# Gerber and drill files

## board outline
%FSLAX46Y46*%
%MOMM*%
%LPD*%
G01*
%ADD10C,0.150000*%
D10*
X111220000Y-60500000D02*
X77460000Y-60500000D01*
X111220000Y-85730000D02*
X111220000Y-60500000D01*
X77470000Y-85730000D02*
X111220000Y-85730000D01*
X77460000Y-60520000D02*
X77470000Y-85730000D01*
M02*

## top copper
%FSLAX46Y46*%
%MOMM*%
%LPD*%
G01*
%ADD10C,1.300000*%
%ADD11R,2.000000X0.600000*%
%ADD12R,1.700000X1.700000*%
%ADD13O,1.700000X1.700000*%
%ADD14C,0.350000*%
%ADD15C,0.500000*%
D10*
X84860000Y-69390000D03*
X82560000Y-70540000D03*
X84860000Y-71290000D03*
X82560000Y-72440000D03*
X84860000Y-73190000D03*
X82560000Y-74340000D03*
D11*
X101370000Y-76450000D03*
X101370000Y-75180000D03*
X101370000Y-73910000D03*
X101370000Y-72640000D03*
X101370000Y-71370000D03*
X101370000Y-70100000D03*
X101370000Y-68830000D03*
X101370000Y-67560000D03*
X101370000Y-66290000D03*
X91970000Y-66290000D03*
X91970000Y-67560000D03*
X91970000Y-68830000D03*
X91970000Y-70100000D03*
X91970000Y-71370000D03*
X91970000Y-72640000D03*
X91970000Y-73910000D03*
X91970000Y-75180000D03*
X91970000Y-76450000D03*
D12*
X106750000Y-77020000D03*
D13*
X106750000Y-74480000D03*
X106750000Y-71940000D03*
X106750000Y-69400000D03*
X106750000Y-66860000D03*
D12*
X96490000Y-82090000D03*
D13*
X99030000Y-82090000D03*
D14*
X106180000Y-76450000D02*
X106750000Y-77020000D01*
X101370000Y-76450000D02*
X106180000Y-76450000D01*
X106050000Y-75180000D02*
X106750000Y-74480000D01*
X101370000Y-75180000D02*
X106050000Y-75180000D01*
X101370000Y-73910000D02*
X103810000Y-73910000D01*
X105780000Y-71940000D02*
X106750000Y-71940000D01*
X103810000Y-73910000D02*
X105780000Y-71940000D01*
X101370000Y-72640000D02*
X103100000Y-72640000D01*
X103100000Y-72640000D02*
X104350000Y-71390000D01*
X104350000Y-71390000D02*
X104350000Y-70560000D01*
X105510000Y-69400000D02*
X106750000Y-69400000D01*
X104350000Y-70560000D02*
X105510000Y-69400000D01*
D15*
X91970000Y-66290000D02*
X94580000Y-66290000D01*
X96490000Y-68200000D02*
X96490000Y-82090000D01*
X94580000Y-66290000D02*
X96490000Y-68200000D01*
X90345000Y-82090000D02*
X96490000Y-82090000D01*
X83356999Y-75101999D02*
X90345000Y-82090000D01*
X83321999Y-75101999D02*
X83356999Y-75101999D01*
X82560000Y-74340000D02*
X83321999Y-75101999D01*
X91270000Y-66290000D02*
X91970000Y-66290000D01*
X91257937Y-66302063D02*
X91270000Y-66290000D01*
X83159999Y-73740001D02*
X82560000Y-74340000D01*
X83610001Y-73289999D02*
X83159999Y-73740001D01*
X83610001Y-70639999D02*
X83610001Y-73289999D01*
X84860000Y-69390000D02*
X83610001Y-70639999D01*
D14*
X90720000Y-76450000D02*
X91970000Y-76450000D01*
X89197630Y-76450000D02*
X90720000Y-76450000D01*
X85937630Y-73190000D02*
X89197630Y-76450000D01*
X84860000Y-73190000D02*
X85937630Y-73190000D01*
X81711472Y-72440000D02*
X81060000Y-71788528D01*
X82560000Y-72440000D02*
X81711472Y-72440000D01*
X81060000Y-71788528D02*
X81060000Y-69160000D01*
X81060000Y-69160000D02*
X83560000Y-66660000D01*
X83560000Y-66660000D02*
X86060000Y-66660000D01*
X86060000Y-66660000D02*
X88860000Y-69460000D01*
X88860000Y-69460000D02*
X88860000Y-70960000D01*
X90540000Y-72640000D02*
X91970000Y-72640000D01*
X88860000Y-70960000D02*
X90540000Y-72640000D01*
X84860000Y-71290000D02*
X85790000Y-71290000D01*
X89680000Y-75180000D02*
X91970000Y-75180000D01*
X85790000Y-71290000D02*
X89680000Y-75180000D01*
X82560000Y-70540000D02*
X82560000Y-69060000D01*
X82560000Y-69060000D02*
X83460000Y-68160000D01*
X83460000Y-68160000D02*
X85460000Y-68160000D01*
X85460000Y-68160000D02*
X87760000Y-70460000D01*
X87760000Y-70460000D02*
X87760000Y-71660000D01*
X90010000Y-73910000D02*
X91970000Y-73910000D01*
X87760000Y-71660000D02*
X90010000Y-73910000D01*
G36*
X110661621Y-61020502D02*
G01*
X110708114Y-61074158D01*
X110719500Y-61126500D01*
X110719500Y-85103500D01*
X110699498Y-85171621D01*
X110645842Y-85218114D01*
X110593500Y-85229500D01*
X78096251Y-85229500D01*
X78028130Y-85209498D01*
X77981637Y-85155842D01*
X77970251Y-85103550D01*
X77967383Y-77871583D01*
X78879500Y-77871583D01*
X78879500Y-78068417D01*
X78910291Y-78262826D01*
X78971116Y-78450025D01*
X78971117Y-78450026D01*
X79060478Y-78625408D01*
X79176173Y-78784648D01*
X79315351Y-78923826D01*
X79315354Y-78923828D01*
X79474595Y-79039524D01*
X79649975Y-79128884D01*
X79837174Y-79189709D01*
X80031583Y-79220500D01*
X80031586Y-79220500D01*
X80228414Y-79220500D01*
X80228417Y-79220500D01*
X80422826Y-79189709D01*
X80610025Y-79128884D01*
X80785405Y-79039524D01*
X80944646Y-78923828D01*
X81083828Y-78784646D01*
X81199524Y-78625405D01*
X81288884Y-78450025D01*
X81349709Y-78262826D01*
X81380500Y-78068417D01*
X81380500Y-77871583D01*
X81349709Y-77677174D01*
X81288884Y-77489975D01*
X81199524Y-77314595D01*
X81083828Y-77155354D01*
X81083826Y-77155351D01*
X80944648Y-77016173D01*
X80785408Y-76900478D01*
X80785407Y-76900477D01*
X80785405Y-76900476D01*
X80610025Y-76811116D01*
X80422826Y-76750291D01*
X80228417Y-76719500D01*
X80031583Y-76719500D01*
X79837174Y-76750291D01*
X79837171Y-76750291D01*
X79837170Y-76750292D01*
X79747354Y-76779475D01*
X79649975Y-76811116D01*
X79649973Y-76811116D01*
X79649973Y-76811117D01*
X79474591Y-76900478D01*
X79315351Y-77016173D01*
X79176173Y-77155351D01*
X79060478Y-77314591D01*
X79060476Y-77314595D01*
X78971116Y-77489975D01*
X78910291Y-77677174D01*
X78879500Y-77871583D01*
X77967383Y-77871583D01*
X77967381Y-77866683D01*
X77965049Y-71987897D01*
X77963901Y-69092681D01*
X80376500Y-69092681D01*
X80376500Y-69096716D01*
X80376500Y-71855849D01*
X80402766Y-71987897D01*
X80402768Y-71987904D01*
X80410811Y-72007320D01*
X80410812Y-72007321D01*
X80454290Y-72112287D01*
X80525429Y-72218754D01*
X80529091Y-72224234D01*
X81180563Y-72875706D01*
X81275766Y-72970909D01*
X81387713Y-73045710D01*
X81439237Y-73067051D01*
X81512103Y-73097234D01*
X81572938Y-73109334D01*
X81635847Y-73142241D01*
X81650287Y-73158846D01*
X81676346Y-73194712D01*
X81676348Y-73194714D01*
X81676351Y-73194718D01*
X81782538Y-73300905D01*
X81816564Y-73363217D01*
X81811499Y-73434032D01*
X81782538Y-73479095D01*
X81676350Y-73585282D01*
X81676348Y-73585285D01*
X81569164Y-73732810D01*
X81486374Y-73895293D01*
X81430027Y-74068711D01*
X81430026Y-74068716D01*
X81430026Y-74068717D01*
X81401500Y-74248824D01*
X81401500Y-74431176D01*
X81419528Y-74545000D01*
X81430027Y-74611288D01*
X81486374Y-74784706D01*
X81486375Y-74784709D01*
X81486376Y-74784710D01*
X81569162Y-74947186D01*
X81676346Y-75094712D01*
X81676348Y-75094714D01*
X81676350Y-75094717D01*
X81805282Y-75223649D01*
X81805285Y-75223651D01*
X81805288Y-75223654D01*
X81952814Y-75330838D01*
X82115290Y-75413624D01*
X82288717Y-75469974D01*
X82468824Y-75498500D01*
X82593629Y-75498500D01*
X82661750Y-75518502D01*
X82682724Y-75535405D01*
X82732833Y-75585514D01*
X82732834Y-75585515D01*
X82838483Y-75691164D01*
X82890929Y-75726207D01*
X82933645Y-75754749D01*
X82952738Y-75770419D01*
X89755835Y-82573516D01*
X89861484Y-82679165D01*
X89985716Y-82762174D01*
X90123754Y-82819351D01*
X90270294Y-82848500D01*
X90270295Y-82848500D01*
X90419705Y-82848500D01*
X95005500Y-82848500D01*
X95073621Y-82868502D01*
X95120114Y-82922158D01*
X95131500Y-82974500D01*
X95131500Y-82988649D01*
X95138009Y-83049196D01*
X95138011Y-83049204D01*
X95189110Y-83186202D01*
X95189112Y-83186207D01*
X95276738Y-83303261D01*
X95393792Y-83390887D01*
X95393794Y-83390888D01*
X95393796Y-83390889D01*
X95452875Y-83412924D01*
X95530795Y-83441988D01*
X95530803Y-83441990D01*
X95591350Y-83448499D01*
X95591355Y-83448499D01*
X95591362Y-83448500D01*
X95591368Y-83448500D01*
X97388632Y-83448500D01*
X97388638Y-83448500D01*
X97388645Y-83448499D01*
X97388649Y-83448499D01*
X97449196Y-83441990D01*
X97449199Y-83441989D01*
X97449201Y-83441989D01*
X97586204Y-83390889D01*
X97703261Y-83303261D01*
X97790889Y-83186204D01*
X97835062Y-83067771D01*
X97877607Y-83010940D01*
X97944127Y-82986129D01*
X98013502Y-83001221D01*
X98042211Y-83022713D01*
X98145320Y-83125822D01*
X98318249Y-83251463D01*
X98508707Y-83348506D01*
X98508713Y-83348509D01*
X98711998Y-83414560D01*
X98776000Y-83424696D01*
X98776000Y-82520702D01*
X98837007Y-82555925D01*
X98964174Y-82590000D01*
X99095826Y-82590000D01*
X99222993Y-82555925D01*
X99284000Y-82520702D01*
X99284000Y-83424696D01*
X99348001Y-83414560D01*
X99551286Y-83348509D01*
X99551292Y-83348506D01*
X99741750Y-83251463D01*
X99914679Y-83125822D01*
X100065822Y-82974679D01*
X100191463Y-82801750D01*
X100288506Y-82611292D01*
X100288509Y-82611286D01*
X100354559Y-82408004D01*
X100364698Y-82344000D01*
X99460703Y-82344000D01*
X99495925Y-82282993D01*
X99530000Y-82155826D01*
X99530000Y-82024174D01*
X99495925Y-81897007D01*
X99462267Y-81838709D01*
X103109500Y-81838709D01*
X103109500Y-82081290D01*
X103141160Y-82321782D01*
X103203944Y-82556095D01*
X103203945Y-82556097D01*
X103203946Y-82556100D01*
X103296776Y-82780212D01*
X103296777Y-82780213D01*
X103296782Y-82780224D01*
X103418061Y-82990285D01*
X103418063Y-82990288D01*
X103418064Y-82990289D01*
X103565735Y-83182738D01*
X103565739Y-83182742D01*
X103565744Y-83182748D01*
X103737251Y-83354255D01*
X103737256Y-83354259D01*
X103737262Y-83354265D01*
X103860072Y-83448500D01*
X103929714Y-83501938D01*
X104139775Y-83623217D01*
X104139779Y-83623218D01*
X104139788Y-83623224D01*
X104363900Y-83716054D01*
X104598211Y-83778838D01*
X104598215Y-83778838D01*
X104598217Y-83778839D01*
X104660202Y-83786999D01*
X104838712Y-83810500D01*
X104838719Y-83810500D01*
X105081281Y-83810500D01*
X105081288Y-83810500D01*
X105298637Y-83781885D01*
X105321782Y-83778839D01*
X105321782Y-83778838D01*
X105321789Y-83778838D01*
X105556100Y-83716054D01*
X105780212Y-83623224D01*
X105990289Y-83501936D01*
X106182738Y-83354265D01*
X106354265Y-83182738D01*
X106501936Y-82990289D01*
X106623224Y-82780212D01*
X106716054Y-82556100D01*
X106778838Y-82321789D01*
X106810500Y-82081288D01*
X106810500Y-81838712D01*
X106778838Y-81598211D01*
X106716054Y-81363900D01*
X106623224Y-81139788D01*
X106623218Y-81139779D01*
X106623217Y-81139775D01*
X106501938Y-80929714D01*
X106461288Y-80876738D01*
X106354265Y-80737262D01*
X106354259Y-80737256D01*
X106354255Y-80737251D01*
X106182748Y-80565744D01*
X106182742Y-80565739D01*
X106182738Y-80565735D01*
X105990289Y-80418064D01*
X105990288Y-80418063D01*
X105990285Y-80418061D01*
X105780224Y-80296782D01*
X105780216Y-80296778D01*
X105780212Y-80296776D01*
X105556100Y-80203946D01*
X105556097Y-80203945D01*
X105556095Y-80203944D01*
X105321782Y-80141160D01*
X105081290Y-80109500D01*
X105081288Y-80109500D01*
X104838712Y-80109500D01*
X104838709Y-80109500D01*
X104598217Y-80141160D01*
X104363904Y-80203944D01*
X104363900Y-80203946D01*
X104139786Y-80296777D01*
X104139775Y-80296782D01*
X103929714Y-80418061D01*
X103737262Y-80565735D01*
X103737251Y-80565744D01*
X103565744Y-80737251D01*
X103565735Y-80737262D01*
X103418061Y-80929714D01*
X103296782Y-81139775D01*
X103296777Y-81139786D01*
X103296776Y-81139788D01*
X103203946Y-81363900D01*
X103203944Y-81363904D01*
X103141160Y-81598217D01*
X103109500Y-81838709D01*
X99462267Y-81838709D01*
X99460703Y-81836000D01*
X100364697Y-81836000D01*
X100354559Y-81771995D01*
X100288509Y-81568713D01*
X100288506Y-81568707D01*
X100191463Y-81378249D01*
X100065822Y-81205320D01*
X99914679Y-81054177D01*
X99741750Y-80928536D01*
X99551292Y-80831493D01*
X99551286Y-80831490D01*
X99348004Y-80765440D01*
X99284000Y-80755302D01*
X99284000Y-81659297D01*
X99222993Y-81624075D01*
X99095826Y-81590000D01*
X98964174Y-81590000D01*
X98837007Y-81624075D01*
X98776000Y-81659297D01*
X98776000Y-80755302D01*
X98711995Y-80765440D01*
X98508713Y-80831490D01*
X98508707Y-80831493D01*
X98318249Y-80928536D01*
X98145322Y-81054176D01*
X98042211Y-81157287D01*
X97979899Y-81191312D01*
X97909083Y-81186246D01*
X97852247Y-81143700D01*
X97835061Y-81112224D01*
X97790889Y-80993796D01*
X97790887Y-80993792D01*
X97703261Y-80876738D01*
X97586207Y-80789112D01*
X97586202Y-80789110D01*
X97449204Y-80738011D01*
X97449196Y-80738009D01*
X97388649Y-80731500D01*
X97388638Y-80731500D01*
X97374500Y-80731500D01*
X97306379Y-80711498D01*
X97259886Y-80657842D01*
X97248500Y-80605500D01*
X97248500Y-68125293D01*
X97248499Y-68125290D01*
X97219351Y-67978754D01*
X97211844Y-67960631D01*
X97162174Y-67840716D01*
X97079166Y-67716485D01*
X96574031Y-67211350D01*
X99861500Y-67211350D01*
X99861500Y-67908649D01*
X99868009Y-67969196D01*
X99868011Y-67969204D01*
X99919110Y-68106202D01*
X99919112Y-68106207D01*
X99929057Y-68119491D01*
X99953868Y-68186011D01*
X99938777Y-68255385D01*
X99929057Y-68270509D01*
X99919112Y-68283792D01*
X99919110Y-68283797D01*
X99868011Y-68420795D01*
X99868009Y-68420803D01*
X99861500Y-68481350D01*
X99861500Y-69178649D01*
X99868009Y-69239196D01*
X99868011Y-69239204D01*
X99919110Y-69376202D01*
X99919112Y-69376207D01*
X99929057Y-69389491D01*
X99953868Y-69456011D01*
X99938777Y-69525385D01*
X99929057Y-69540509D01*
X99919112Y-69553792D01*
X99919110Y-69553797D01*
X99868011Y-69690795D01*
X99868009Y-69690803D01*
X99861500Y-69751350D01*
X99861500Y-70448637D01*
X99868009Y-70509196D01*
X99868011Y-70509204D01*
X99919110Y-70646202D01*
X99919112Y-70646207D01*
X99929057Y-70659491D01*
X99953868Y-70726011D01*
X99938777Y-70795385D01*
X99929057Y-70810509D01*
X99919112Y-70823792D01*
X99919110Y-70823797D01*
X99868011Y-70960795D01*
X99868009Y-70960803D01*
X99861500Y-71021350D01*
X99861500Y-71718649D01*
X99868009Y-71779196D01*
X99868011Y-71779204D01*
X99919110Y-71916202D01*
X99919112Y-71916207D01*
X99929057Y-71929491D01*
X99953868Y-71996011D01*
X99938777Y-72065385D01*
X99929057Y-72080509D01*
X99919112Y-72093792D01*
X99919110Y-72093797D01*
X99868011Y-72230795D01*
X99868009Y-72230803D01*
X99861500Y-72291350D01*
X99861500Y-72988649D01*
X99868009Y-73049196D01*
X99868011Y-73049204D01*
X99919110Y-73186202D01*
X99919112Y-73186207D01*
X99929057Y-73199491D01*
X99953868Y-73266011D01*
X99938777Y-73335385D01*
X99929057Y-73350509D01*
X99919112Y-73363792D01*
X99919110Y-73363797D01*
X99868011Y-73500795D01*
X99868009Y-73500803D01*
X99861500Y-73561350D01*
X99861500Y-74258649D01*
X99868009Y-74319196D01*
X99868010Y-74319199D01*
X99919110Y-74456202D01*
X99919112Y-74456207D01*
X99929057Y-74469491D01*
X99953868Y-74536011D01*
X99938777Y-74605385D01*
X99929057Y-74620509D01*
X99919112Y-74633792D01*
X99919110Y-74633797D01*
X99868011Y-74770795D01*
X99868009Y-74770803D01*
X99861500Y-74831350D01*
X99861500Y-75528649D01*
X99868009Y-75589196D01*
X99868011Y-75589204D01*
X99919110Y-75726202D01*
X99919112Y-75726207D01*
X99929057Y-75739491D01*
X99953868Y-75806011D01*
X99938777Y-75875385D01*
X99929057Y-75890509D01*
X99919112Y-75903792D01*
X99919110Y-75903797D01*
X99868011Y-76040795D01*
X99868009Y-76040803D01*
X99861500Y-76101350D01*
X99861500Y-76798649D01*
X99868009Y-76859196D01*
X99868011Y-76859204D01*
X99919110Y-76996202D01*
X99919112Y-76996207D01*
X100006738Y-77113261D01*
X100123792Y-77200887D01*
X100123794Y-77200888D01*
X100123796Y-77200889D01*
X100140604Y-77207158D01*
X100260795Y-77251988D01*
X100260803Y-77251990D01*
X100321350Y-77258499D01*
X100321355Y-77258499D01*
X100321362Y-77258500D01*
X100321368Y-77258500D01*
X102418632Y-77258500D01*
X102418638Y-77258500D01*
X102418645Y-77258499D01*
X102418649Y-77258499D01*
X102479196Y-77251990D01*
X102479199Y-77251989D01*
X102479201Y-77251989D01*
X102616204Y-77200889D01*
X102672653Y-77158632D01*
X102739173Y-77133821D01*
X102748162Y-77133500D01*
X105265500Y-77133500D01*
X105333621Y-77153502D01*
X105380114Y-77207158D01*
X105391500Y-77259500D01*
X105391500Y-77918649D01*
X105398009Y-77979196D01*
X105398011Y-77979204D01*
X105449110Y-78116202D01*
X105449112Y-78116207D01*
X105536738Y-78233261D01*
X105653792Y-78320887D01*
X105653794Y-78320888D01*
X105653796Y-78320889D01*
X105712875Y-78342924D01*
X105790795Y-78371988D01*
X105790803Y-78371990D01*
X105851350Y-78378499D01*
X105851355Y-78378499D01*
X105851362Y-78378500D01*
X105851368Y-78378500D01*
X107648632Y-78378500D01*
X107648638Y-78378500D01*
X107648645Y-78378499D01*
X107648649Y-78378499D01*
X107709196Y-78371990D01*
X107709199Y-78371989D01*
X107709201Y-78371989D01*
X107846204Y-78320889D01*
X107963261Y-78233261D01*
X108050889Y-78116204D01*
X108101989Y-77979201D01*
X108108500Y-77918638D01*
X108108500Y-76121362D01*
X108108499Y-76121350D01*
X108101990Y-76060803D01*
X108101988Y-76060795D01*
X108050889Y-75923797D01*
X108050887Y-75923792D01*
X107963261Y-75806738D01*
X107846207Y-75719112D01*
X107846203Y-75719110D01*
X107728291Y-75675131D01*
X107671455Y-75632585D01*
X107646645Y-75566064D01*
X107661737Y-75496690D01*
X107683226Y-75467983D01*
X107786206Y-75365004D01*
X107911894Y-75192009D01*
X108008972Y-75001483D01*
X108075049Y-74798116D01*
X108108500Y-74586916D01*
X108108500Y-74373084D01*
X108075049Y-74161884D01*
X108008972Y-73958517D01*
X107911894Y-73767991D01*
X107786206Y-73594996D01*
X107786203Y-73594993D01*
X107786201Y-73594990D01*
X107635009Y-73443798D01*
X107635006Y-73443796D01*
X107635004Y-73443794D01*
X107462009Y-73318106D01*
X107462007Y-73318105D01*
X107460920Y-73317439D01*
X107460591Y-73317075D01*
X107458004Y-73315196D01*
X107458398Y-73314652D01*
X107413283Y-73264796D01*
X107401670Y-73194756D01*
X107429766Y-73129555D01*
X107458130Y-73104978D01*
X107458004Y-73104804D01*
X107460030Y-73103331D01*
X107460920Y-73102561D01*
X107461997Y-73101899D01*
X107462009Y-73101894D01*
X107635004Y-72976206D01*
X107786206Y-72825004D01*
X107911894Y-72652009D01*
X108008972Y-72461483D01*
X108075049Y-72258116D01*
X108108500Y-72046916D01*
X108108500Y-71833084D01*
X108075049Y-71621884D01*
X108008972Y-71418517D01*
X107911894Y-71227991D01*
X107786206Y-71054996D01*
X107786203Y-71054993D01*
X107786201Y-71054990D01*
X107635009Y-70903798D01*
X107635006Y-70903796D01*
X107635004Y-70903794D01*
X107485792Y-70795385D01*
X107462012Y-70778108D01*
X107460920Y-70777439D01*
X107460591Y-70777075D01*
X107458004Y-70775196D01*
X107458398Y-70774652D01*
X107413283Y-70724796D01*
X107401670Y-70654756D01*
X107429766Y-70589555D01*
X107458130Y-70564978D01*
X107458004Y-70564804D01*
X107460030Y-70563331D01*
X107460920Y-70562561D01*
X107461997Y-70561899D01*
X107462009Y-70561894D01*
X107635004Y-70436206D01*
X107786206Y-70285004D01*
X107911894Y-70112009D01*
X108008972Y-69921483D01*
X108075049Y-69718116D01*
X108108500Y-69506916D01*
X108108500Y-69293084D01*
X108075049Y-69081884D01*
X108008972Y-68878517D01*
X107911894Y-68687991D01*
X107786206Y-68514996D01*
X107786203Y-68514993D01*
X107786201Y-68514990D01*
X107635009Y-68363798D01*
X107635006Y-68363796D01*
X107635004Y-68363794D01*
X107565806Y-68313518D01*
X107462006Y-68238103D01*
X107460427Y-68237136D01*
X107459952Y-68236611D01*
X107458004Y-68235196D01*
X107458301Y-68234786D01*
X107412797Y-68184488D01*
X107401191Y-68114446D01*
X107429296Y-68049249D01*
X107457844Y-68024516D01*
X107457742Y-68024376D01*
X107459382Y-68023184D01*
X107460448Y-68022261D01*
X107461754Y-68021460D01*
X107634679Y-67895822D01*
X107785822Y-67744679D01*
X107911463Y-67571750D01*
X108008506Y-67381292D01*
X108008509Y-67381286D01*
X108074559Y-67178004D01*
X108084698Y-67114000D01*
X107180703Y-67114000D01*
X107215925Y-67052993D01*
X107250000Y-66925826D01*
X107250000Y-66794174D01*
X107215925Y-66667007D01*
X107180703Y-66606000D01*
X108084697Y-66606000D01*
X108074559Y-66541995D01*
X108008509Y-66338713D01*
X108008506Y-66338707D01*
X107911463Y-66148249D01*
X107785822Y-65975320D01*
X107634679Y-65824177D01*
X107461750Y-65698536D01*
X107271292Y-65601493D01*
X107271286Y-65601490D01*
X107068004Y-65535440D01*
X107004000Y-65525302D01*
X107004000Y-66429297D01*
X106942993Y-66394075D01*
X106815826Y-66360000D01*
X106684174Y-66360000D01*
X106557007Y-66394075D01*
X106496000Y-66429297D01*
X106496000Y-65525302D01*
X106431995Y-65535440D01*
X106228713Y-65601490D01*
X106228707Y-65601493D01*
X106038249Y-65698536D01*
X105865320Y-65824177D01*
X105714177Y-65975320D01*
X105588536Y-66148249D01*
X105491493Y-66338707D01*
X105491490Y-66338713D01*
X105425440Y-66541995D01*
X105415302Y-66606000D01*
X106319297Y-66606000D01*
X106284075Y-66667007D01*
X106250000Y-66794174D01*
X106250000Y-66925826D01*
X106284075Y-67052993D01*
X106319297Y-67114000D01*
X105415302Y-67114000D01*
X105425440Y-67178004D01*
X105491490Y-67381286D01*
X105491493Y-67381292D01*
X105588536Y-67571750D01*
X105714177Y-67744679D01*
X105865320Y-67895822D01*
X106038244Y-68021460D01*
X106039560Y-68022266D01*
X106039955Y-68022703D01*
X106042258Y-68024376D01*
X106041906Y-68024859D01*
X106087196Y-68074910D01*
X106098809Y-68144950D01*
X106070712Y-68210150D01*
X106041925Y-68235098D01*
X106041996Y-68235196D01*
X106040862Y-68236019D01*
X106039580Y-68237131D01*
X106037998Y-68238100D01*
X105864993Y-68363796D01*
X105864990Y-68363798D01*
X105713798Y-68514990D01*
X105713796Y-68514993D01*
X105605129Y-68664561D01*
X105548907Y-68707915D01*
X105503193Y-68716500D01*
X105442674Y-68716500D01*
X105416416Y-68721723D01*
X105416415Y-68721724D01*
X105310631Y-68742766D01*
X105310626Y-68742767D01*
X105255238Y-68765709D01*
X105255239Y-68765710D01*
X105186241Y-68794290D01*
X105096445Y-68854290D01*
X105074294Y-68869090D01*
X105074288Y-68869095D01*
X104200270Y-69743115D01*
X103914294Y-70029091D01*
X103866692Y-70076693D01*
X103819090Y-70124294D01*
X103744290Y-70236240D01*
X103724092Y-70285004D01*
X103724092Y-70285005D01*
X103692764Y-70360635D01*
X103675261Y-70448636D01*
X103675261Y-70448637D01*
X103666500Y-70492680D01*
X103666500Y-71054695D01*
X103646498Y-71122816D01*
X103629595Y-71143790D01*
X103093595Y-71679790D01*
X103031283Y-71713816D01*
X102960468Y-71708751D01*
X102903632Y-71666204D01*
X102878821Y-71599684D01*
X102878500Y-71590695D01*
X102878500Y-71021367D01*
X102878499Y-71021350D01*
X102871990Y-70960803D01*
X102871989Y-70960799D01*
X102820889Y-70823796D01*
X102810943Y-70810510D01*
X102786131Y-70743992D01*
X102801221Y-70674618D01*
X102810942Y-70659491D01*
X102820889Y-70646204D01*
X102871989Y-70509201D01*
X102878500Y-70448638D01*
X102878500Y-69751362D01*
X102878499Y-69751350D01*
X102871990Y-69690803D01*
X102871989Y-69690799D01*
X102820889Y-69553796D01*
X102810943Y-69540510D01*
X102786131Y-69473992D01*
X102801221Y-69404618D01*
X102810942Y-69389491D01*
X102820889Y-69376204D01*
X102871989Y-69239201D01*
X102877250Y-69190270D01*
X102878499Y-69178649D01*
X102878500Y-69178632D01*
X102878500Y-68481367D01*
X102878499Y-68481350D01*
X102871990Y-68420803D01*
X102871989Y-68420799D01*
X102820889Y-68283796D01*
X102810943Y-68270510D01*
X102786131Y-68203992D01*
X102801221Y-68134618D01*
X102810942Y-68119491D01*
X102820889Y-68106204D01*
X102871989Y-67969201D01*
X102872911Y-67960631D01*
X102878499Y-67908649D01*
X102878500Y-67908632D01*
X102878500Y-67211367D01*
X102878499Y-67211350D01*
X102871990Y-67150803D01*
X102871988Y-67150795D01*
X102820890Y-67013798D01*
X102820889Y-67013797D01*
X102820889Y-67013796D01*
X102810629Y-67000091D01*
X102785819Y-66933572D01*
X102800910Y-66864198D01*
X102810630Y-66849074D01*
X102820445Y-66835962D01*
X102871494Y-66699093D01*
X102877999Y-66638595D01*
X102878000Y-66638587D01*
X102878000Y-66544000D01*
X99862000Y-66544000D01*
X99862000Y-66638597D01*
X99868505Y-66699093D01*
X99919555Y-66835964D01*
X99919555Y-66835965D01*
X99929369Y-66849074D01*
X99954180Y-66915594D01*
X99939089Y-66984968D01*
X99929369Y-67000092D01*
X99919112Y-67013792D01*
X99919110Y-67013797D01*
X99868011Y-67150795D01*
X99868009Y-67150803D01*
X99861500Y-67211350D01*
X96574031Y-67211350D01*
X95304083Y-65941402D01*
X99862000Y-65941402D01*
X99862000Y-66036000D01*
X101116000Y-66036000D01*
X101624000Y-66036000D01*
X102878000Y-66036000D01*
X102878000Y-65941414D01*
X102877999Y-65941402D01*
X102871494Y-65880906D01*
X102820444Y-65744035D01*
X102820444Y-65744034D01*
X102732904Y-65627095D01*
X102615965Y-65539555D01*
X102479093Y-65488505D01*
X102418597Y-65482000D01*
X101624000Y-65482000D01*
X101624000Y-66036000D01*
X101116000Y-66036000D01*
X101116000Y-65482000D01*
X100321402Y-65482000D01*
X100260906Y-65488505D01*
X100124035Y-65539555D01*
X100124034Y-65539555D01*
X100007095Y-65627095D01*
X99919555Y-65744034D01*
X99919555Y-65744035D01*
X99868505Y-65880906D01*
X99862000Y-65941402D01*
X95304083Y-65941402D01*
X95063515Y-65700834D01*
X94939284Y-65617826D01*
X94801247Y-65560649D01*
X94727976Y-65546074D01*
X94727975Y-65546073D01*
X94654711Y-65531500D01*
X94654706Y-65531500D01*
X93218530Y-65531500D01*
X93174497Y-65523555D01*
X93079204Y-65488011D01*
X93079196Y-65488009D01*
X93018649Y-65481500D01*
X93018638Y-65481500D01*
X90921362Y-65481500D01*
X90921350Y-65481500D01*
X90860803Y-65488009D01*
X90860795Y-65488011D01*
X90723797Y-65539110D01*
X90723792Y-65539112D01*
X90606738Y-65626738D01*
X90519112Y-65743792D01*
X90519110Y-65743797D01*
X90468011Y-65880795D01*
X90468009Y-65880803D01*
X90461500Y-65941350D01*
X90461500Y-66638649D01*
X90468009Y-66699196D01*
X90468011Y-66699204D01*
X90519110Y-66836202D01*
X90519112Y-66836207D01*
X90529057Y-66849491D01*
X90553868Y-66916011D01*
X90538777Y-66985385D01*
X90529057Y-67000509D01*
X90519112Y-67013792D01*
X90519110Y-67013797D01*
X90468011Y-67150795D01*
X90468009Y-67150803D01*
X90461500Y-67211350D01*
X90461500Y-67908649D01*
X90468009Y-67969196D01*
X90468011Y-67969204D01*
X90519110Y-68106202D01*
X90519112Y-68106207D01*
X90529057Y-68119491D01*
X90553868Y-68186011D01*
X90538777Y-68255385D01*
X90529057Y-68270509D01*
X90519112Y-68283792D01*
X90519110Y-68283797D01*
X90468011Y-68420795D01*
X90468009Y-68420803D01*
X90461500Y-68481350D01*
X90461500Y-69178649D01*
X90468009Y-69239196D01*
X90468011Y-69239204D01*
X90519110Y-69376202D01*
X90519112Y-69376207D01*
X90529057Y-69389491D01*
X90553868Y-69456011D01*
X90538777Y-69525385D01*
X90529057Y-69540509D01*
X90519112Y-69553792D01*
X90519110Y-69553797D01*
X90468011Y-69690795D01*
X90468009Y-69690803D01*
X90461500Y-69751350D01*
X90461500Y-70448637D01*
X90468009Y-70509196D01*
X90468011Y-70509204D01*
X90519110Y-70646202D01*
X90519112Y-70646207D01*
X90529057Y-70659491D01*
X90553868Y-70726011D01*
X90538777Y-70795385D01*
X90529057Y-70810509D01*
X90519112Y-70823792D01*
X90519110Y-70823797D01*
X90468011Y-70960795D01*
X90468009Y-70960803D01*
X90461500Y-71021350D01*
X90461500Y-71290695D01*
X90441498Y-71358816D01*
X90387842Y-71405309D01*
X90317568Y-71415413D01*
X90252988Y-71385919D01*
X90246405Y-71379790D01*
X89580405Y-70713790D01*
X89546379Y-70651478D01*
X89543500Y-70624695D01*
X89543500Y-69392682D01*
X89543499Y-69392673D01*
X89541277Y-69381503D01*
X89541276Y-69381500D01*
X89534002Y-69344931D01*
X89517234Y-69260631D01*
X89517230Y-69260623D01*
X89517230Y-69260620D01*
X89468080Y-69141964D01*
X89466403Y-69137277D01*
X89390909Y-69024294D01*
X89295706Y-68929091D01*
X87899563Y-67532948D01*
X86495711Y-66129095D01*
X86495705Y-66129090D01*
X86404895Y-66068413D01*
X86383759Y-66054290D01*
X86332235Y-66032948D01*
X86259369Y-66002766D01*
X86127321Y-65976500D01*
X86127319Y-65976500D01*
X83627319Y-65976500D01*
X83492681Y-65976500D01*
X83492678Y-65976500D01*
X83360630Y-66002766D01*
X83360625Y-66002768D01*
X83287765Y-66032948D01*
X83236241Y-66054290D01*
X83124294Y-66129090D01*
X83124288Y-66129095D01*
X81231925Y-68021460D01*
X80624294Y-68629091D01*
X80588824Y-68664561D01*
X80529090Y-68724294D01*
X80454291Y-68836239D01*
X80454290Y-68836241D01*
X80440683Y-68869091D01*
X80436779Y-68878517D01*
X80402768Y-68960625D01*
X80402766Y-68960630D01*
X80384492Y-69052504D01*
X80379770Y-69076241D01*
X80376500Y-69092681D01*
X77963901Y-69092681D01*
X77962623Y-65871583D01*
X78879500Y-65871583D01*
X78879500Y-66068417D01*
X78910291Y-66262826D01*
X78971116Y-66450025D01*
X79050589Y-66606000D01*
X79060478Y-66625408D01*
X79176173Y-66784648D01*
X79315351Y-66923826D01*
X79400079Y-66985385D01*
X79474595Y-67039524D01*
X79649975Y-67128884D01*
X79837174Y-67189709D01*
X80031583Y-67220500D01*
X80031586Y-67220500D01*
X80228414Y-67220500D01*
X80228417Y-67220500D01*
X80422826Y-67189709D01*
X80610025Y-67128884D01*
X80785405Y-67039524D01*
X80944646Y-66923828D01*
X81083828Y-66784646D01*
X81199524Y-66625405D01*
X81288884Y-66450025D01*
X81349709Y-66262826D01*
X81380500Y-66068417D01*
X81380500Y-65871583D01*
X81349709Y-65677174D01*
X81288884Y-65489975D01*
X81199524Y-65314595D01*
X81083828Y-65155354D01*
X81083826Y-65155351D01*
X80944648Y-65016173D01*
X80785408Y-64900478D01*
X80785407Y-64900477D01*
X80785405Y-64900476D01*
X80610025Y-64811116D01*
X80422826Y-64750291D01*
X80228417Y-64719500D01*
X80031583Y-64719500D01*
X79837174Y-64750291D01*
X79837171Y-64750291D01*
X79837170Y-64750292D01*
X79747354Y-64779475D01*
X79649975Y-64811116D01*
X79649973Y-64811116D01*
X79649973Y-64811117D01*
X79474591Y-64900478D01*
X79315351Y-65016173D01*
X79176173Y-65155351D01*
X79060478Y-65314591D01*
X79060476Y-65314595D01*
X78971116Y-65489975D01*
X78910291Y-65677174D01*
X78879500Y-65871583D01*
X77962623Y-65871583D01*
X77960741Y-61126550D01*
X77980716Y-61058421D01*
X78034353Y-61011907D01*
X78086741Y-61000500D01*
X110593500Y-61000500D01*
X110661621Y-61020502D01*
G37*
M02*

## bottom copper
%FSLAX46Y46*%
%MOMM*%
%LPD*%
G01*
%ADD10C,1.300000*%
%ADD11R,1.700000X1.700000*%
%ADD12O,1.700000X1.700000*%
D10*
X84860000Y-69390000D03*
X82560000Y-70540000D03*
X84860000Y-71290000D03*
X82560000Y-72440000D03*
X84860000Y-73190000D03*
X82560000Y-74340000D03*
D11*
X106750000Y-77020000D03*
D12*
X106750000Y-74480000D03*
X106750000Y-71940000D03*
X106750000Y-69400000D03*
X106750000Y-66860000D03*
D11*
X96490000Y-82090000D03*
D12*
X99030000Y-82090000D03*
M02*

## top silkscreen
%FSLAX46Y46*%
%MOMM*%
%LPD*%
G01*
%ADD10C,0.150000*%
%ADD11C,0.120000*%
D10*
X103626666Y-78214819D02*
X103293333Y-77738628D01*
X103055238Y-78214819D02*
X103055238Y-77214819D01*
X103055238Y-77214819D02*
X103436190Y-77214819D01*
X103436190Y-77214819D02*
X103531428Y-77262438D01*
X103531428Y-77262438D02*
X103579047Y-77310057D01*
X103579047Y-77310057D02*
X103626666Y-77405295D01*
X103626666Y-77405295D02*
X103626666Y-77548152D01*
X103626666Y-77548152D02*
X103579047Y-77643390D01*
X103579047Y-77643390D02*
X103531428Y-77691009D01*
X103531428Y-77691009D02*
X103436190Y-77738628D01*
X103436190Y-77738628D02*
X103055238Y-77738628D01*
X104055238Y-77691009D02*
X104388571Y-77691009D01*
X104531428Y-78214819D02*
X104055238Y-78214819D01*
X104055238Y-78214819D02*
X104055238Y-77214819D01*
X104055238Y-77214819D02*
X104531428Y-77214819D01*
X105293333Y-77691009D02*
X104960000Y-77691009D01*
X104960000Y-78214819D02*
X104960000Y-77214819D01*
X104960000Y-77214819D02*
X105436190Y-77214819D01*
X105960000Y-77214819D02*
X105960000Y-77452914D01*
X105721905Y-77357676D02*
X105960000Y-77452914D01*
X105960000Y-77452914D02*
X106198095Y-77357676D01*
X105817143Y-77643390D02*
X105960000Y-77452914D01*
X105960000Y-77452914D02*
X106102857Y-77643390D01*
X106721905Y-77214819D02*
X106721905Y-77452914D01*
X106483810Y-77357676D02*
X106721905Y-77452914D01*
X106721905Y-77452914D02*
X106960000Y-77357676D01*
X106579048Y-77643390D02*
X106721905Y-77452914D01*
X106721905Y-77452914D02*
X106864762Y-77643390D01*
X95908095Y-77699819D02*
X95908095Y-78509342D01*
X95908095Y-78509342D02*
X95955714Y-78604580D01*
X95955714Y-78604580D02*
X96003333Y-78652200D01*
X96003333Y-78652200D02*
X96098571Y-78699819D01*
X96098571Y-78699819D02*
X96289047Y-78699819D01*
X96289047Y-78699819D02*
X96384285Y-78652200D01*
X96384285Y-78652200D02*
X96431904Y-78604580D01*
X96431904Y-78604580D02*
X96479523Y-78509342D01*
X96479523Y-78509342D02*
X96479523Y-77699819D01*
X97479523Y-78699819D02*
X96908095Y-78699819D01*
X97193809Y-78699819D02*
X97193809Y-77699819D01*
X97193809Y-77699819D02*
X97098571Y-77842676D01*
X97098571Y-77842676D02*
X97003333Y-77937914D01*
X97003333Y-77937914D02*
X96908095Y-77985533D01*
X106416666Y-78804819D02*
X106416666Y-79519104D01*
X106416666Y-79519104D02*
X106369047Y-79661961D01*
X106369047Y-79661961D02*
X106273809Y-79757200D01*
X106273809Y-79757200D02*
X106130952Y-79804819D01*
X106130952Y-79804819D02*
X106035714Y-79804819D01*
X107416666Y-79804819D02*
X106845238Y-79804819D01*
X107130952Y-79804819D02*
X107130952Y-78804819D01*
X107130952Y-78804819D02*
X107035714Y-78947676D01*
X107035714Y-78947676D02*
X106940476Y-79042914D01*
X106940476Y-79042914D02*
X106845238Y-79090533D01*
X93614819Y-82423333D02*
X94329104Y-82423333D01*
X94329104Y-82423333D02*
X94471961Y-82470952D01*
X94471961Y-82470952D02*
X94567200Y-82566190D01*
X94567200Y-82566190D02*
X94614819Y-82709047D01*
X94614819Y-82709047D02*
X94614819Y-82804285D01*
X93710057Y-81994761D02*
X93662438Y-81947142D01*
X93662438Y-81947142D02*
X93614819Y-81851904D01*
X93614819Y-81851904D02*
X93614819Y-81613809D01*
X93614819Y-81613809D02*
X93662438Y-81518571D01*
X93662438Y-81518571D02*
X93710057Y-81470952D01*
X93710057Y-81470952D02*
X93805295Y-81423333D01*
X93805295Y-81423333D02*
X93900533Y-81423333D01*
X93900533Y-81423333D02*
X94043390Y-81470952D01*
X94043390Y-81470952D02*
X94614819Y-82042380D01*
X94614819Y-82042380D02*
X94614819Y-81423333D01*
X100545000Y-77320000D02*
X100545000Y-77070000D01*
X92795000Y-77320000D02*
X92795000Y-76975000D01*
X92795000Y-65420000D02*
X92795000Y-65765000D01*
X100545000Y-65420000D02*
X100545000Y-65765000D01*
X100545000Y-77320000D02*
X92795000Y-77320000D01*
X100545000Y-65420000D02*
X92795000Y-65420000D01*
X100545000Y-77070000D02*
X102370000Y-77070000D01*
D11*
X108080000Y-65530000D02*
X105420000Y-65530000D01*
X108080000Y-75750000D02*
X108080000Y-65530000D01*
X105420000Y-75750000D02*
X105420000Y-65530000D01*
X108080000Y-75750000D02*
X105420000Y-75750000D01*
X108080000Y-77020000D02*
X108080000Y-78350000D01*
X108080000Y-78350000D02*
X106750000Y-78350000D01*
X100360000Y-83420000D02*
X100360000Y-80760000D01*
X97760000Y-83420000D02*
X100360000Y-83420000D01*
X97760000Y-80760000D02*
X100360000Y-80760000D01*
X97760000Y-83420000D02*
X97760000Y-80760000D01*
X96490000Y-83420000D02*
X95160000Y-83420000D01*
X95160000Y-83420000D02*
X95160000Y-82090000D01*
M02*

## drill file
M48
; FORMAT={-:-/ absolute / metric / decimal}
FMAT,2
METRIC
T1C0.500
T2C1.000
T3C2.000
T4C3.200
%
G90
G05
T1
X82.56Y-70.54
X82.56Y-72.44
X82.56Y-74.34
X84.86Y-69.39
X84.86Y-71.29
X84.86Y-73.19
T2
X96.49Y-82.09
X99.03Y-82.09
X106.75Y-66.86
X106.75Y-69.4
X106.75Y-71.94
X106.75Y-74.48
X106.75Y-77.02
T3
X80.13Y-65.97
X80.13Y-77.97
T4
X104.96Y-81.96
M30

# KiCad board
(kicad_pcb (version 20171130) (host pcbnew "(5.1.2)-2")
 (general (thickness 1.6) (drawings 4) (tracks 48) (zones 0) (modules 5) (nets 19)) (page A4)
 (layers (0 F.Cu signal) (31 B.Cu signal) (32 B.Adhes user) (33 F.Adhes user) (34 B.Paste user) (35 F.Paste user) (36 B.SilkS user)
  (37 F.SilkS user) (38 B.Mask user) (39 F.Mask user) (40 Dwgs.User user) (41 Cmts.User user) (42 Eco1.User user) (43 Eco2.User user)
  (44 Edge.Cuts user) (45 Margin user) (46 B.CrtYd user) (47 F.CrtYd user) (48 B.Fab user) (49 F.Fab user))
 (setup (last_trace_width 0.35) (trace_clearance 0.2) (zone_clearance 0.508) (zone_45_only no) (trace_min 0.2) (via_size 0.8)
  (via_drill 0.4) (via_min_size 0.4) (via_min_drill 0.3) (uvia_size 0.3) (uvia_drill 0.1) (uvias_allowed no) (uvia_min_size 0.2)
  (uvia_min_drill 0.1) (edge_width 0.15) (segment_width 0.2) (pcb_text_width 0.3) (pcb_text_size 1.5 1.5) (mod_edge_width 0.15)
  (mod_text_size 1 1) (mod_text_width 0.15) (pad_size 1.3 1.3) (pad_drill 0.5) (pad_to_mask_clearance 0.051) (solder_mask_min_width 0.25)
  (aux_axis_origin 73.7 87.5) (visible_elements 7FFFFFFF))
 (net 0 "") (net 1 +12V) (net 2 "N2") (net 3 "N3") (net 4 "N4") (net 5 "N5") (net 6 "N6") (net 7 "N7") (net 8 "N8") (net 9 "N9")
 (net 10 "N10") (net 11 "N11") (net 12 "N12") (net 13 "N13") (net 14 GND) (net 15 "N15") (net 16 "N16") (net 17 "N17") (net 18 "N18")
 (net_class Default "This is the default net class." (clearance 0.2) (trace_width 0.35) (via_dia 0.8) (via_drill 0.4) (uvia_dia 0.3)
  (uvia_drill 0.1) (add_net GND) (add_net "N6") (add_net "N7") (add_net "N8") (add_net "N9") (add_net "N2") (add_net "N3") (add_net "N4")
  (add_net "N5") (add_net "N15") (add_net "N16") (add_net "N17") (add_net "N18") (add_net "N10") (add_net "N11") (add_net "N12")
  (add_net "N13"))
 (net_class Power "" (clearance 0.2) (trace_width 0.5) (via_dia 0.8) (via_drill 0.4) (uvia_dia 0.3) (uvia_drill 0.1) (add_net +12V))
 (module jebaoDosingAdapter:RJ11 (layer B.Cu) (at 87.63 77.47 180)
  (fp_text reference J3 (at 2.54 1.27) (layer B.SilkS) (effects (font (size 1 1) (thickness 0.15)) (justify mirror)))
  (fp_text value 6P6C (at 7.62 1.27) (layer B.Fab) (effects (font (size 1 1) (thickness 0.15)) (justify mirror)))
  (pad 1 thru_hole circle (at 2.77 8.08 180) (size 1.3 1.3) (drill 0.5) (layers *.Cu *.Mask) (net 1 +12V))
  (pad 2 thru_hole circle (at 5.07 6.93 180) (size 1.3 1.3) (drill 0.5) (layers *.Cu *.Mask) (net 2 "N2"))
  (pad 3 thru_hole circle (at 2.77 6.18 180) (size 1.3 1.3) (drill 0.5) (layers *.Cu *.Mask) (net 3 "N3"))
  (pad 4 thru_hole circle (at 5.07 5.03 180) (size 1.3 1.3) (drill 0.5) (layers *.Cu *.Mask) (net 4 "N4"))
  (pad 5 thru_hole circle (at 2.77 4.28 180) (size 1.3 1.3) (drill 0.5) (layers *.Cu *.Mask) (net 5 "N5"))
  (pad 6 thru_hole circle (at 5.07 3.13 180) (size 1.3 1.3) (drill 0.5) (layers *.Cu *.Mask) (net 1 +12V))
  (pad "" np_thru_hole circle (at 7.5 -0.5 180) (size 2 2) (drill 2) (layers *.Cu *.Mask))
  (pad "" np_thru_hole circle (at 7.5 11.5 180) (size 2 2) (drill 2) (layers *.Cu *.Mask)))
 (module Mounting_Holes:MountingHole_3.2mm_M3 (layer F.Cu) (at 104.96 81.96)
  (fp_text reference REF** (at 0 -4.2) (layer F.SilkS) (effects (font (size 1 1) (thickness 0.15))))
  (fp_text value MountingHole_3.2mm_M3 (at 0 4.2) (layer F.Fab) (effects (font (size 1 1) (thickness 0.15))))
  (pad 1 np_thru_hole circle (at 0 0) (size 3.2 3.2) (drill 3.2) (layers *.Cu *.Mask)))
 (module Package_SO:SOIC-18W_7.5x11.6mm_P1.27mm (layer F.Cu) (at 96.67 71.37 180)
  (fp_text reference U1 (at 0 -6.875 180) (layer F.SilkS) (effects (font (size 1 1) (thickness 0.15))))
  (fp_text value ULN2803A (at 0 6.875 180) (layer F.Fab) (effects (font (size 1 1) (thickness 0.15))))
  (fp_line (start -3.875 -5.95) (end -3.875 -5.7) (layer F.SilkS) (width 0.15))
  (fp_line (start 3.875 -5.95) (end 3.875 -5.605) (layer F.SilkS) (width 0.15))
  (fp_line (start 3.875 5.95) (end 3.875 5.605) (layer F.SilkS) (width 0.15))
  (fp_line (start -3.875 5.95) (end -3.875 5.605) (layer F.SilkS) (width 0.15))
  (fp_line (start -3.875 -5.95) (end 3.875 -5.95) (layer F.SilkS) (width 0.15))
  (fp_line (start -3.875 5.95) (end 3.875 5.95) (layer F.SilkS) (width 0.15))
  (fp_line (start -3.875 -5.7) (end -5.7 -5.7) (layer F.SilkS) (width 0.15))
  (pad 1 smd rect (at -4.7 -5.08 180) (size 2 0.6) (layers F.Cu F.Paste F.Mask) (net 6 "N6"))
  (pad 2 smd rect (at -4.7 -3.81 180) (size 2 0.6) (layers F.Cu F.Paste F.Mask) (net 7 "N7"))
  (pad 3 smd rect (at -4.7 -2.54 180) (size 2 0.6) (layers F.Cu F.Paste F.Mask) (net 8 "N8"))
  (pad 4 smd rect (at -4.7 -1.27 180) (size 2 0.6) (layers F.Cu F.Paste F.Mask) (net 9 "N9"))
  (pad 5 smd rect (at -4.7 0 180) (size 2 0.6) (layers F.Cu F.Paste F.Mask) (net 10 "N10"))
  (pad 6 smd rect (at -4.7 1.27 180) (size 2 0.6) (layers F.Cu F.Paste F.Mask) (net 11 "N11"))
  (pad 7 smd rect (at -4.7 2.54 180) (size 2 0.6) (layers F.Cu F.Paste F.Mask) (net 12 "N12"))
  (pad 8 smd rect (at -4.7 3.81 180) (size 2 0.6) (layers F.Cu F.Paste F.Mask) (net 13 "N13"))
  (pad 9 smd rect (at -4.7 5.08 180) (size 2 0.6) (layers F.Cu F.Paste F.Mask) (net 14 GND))
  (pad 10 smd rect (at 4.7 5.08 180) (size 2 0.6) (layers F.Cu F.Paste F.Mask) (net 1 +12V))
  (pad 11 smd rect (at 4.7 3.81 180) (size 2 0.6) (layers F.Cu F.Paste F.Mask) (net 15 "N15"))
  (pad 12 smd rect (at 4.7 2.54 180) (size 2 0.6) (layers F.Cu F.Paste F.Mask) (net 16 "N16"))
  (pad 13 smd rect (at 4.7 1.27 180) (size 2 0.6) (layers F.Cu F.Paste F.Mask) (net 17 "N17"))
  (pad 14 smd rect (at 4.7 0 180) (size 2 0.6) (layers F.Cu F.Paste F.Mask) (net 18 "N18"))
  (pad 15 smd rect (at 4.7 -1.27 180) (size 2 0.6) (layers F.Cu F.Paste F.Mask) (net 4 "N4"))
  (pad 16 smd rect (at 4.7 -2.54 180) (size 2 0.6) (layers F.Cu F.Paste F.Mask) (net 2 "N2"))
  (pad 17 smd rect (at 4.7 -3.81 180) (size 2 0.6) (layers F.Cu F.Paste F.Mask) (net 3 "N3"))
  (pad 18 smd rect (at 4.7 -5.08 180) (size 2 0.6) (layers F.Cu F.Paste F.Mask) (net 5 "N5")))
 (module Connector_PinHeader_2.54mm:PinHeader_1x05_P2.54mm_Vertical (layer F.Cu) (at 106.75 77.02 180)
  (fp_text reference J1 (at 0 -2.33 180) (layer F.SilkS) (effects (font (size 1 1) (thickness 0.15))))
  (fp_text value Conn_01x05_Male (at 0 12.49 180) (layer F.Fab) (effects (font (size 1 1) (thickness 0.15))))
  (fp_line (start -1.33 11.49) (end 1.33 11.49) (layer F.SilkS) (width 0.12))
  (fp_line (start -1.33 1.27) (end -1.33 11.49) (layer F.SilkS) (width 0.12))
  (fp_line (start 1.33 1.27) (end 1.33 11.49) (layer F.SilkS) (width 0.12))
  (fp_line (start -1.33 1.27) (end 1.33 1.27) (layer F.SilkS) (width 0.12))
  (fp_line (start -1.33 0) (end -1.33 -1.33) (layer F.SilkS) (width 0.12))
  (fp_line (start -1.33 -1.33) (end 0 -1.33) (layer F.SilkS) (width 0.12))
  (pad 1 thru_hole rect (at 0 0 180) (size 1.7 1.7) (drill 1) (layers *.Cu *.Mask) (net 6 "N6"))
  (pad 2 thru_hole oval (at 0 2.54 180) (size 1.7 1.7) (drill 1) (layers *.Cu *.Mask) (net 7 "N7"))
  (pad 3 thru_hole oval (at 0 5.08 180) (size 1.7 1.7) (drill 1) (layers *.Cu *.Mask) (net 8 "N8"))
  (pad 4 thru_hole oval (at 0 7.62 180) (size 1.7 1.7) (drill 1) (layers *.Cu *.Mask) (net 9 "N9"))
  (pad 5 thru_hole oval (at 0 10.16 180) (size 1.7 1.7) (drill 1) (layers *.Cu *.Mask) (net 14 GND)))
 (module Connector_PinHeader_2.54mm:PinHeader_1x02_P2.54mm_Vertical (layer F.Cu) (at 96.49 82.09 90)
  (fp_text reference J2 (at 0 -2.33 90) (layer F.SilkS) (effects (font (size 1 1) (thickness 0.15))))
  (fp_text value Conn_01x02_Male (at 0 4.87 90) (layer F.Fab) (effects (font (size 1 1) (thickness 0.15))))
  (fp_line (start -1.33 3.87) (end 1.33 3.87) (layer F.SilkS) (width 0.12))
  (fp_line (start -1.33 1.27) (end -1.33 3.87) (layer F.SilkS) (width 0.12))
  (fp_line (start 1.33 1.27) (end 1.33 3.87) (layer F.SilkS) (width 0.12))
  (fp_line (start -1.33 1.27) (end 1.33 1.27) (layer F.SilkS) (width 0.12))
  (fp_line (start -1.33 0) (end -1.33 -1.33) (layer F.SilkS) (width 0.12))
  (fp_line (start -1.33 -1.33) (end 0 -1.33) (layer F.SilkS) (width 0.12))
  (pad 1 thru_hole rect (at 0 0 90) (size 1.7 1.7) (drill 1) (layers *.Cu *.Mask) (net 1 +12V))
  (pad 2 thru_hole oval (at 0 2.54 90) (size 1.7 1.7) (drill 1) (layers *.Cu *.Mask) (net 14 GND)))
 (gr_line (start 111.22 60.5) (end 77.46 60.5) (layer Edge.Cuts) (width 0.15))
 (gr_line (start 111.22 85.73) (end 111.22 60.5) (layer Edge.Cuts) (width 0.15))
 (gr_line (start 77.47 85.73) (end 111.22 85.73) (layer Edge.Cuts) (width 0.15))
 (gr_line (start 77.46 60.52) (end 77.47 85.73) (layer Edge.Cuts) (width 0.15))
 (segment (start 106.18 76.45) (end 106.75 77.02) (width 0.35) (layer F.Cu) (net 6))
 (segment (start 101.37 76.45) (end 106.18 76.45) (width 0.35) (layer F.Cu) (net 6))
 (segment (start 106.05 75.18) (end 106.75 74.48) (width 0.35) (layer F.Cu) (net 7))
 (segment (start 101.37 75.18) (end 106.05 75.18) (width 0.35) (layer F.Cu) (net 7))
 (segment (start 101.37 73.91) (end 103.81 73.91) (width 0.35) (layer F.Cu) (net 8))
 (segment (start 105.78 71.94) (end 106.75 71.94) (width 0.35) (layer F.Cu) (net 8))
 (segment (start 103.81 73.91) (end 105.78 71.94) (width 0.35) (layer F.Cu) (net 8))
 (segment (start 101.37 72.64) (end 103.1 72.64) (width 0.35) (layer F.Cu) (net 9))
 (segment (start 103.1 72.64) (end 104.35 71.39) (width 0.35) (layer F.Cu) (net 9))
 (segment (start 104.35 71.39) (end 104.35 70.56) (width 0.35) (layer F.Cu) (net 9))
 (segment (start 105.51 69.4) (end 106.75 69.4) (width 0.35) (layer F.Cu) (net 9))
 (segment (start 104.35 70.56) (end 105.51 69.4) (width 0.35) (layer F.Cu) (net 9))
 (segment (start 91.97 66.29) (end 94.58 66.29) (width 0.5) (layer F.Cu) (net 1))
 (segment (start 96.49 68.2) (end 96.49 82.09) (width 0.5) (layer F.Cu) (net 1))
 (segment (start 94.58 66.29) (end 96.49 68.2) (width 0.5) (layer F.Cu) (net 1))
 (segment (start 90.345 82.09) (end 96.49 82.09) (width 0.5) (layer F.Cu) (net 1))
 (segment (start 83.356999 75.101999) (end 90.345 82.09) (width 0.5) (layer F.Cu) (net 1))
 (segment (start 83.321999 75.101999) (end 83.356999 75.101999) (width 0.5) (layer F.Cu) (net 1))
 (segment (start 82.56 74.34) (end 83.321999 75.101999) (width 0.5) (layer F.Cu) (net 1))
 (segment (start 91.27 66.29) (end 91.97 66.29) (width 0.5) (layer F.Cu) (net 1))
 (segment (start 91.257937 66.302063) (end 91.27 66.29) (width 0.5) (layer F.Cu) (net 1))
 (segment (start 83.159999 73.740001) (end 82.56 74.34) (width 0.5) (layer F.Cu) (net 1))
 (segment (start 83.610001 73.289999) (end 83.159999 73.740001) (width 0.5) (layer F.Cu) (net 1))
 (segment (start 83.610001 70.639999) (end 83.610001 73.289999) (width 0.5) (layer F.Cu) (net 1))
 (segment (start 84.86 69.39) (end 83.610001 70.639999) (width 0.5) (layer F.Cu) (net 1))
 (segment (start 90.72 76.45) (end 91.97 76.45) (width 0.35) (layer F.Cu) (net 5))
 (segment (start 89.19763 76.45) (end 90.72 76.45) (width 0.35) (layer F.Cu) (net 5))
 (segment (start 85.93763 73.19) (end 89.19763 76.45) (width 0.35) (layer F.Cu) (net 5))
 (segment (start 84.86 73.19) (end 85.93763 73.19) (width 0.35) (layer F.Cu) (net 5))
 (segment (start 81.711472 72.44) (end 81.06 71.788528) (width 0.35) (layer F.Cu) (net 4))
 (segment (start 82.56 72.44) (end 81.711472 72.44) (width 0.35) (layer F.Cu) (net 4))
 (segment (start 81.06 71.788528) (end 81.06 69.16) (width 0.35) (layer F.Cu) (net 4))
 (segment (start 81.06 69.16) (end 83.56 66.66) (width 0.35) (layer F.Cu) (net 4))
 (segment (start 83.56 66.66) (end 86.06 66.66) (width 0.35) (layer F.Cu) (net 4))
 (segment (start 86.06 66.66) (end 88.86 69.46) (width 0.35) (layer F.Cu) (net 4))
 (segment (start 88.86 69.46) (end 88.86 70.96) (width 0.35) (layer F.Cu) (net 4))
 (segment (start 90.54 72.64) (end 91.97 72.64) (width 0.35) (layer F.Cu) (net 4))
 (segment (start 88.86 70.96) (end 90.54 72.64) (width 0.35) (layer F.Cu) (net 4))
 (segment (start 84.86 71.29) (end 85.79 71.29) (width 0.35) (layer F.Cu) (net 3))
 (segment (start 89.68 75.18) (end 91.97 75.18) (width 0.35) (layer F.Cu) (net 3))
 (segment (start 85.79 71.29) (end 89.68 75.18) (width 0.35) (layer F.Cu) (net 3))
 (segment (start 82.56 70.54) (end 82.56 69.06) (width 0.35) (layer F.Cu) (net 2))
 (segment (start 82.56 69.06) (end 83.46 68.16) (width 0.35) (layer F.Cu) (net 2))
 (segment (start 83.46 68.16) (end 85.46 68.16) (width 0.35) (layer F.Cu) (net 2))
 (segment (start 85.46 68.16) (end 87.76 70.46) (width 0.35) (layer F.Cu) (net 2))
 (segment (start 87.76 70.46) (end 87.76 71.66) (width 0.35) (layer F.Cu) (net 2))
 (segment (start 90.01 73.91) (end 91.97 73.91) (width 0.35) (layer F.Cu) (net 2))
 (segment (start 87.76 71.66) (end 90.01 73.91) (width 0.35) (layer F.Cu) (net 2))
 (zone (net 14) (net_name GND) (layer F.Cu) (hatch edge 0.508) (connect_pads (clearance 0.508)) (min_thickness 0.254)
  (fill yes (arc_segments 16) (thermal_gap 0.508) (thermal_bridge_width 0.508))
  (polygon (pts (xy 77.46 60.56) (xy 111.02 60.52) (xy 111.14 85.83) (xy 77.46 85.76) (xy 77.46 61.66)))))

